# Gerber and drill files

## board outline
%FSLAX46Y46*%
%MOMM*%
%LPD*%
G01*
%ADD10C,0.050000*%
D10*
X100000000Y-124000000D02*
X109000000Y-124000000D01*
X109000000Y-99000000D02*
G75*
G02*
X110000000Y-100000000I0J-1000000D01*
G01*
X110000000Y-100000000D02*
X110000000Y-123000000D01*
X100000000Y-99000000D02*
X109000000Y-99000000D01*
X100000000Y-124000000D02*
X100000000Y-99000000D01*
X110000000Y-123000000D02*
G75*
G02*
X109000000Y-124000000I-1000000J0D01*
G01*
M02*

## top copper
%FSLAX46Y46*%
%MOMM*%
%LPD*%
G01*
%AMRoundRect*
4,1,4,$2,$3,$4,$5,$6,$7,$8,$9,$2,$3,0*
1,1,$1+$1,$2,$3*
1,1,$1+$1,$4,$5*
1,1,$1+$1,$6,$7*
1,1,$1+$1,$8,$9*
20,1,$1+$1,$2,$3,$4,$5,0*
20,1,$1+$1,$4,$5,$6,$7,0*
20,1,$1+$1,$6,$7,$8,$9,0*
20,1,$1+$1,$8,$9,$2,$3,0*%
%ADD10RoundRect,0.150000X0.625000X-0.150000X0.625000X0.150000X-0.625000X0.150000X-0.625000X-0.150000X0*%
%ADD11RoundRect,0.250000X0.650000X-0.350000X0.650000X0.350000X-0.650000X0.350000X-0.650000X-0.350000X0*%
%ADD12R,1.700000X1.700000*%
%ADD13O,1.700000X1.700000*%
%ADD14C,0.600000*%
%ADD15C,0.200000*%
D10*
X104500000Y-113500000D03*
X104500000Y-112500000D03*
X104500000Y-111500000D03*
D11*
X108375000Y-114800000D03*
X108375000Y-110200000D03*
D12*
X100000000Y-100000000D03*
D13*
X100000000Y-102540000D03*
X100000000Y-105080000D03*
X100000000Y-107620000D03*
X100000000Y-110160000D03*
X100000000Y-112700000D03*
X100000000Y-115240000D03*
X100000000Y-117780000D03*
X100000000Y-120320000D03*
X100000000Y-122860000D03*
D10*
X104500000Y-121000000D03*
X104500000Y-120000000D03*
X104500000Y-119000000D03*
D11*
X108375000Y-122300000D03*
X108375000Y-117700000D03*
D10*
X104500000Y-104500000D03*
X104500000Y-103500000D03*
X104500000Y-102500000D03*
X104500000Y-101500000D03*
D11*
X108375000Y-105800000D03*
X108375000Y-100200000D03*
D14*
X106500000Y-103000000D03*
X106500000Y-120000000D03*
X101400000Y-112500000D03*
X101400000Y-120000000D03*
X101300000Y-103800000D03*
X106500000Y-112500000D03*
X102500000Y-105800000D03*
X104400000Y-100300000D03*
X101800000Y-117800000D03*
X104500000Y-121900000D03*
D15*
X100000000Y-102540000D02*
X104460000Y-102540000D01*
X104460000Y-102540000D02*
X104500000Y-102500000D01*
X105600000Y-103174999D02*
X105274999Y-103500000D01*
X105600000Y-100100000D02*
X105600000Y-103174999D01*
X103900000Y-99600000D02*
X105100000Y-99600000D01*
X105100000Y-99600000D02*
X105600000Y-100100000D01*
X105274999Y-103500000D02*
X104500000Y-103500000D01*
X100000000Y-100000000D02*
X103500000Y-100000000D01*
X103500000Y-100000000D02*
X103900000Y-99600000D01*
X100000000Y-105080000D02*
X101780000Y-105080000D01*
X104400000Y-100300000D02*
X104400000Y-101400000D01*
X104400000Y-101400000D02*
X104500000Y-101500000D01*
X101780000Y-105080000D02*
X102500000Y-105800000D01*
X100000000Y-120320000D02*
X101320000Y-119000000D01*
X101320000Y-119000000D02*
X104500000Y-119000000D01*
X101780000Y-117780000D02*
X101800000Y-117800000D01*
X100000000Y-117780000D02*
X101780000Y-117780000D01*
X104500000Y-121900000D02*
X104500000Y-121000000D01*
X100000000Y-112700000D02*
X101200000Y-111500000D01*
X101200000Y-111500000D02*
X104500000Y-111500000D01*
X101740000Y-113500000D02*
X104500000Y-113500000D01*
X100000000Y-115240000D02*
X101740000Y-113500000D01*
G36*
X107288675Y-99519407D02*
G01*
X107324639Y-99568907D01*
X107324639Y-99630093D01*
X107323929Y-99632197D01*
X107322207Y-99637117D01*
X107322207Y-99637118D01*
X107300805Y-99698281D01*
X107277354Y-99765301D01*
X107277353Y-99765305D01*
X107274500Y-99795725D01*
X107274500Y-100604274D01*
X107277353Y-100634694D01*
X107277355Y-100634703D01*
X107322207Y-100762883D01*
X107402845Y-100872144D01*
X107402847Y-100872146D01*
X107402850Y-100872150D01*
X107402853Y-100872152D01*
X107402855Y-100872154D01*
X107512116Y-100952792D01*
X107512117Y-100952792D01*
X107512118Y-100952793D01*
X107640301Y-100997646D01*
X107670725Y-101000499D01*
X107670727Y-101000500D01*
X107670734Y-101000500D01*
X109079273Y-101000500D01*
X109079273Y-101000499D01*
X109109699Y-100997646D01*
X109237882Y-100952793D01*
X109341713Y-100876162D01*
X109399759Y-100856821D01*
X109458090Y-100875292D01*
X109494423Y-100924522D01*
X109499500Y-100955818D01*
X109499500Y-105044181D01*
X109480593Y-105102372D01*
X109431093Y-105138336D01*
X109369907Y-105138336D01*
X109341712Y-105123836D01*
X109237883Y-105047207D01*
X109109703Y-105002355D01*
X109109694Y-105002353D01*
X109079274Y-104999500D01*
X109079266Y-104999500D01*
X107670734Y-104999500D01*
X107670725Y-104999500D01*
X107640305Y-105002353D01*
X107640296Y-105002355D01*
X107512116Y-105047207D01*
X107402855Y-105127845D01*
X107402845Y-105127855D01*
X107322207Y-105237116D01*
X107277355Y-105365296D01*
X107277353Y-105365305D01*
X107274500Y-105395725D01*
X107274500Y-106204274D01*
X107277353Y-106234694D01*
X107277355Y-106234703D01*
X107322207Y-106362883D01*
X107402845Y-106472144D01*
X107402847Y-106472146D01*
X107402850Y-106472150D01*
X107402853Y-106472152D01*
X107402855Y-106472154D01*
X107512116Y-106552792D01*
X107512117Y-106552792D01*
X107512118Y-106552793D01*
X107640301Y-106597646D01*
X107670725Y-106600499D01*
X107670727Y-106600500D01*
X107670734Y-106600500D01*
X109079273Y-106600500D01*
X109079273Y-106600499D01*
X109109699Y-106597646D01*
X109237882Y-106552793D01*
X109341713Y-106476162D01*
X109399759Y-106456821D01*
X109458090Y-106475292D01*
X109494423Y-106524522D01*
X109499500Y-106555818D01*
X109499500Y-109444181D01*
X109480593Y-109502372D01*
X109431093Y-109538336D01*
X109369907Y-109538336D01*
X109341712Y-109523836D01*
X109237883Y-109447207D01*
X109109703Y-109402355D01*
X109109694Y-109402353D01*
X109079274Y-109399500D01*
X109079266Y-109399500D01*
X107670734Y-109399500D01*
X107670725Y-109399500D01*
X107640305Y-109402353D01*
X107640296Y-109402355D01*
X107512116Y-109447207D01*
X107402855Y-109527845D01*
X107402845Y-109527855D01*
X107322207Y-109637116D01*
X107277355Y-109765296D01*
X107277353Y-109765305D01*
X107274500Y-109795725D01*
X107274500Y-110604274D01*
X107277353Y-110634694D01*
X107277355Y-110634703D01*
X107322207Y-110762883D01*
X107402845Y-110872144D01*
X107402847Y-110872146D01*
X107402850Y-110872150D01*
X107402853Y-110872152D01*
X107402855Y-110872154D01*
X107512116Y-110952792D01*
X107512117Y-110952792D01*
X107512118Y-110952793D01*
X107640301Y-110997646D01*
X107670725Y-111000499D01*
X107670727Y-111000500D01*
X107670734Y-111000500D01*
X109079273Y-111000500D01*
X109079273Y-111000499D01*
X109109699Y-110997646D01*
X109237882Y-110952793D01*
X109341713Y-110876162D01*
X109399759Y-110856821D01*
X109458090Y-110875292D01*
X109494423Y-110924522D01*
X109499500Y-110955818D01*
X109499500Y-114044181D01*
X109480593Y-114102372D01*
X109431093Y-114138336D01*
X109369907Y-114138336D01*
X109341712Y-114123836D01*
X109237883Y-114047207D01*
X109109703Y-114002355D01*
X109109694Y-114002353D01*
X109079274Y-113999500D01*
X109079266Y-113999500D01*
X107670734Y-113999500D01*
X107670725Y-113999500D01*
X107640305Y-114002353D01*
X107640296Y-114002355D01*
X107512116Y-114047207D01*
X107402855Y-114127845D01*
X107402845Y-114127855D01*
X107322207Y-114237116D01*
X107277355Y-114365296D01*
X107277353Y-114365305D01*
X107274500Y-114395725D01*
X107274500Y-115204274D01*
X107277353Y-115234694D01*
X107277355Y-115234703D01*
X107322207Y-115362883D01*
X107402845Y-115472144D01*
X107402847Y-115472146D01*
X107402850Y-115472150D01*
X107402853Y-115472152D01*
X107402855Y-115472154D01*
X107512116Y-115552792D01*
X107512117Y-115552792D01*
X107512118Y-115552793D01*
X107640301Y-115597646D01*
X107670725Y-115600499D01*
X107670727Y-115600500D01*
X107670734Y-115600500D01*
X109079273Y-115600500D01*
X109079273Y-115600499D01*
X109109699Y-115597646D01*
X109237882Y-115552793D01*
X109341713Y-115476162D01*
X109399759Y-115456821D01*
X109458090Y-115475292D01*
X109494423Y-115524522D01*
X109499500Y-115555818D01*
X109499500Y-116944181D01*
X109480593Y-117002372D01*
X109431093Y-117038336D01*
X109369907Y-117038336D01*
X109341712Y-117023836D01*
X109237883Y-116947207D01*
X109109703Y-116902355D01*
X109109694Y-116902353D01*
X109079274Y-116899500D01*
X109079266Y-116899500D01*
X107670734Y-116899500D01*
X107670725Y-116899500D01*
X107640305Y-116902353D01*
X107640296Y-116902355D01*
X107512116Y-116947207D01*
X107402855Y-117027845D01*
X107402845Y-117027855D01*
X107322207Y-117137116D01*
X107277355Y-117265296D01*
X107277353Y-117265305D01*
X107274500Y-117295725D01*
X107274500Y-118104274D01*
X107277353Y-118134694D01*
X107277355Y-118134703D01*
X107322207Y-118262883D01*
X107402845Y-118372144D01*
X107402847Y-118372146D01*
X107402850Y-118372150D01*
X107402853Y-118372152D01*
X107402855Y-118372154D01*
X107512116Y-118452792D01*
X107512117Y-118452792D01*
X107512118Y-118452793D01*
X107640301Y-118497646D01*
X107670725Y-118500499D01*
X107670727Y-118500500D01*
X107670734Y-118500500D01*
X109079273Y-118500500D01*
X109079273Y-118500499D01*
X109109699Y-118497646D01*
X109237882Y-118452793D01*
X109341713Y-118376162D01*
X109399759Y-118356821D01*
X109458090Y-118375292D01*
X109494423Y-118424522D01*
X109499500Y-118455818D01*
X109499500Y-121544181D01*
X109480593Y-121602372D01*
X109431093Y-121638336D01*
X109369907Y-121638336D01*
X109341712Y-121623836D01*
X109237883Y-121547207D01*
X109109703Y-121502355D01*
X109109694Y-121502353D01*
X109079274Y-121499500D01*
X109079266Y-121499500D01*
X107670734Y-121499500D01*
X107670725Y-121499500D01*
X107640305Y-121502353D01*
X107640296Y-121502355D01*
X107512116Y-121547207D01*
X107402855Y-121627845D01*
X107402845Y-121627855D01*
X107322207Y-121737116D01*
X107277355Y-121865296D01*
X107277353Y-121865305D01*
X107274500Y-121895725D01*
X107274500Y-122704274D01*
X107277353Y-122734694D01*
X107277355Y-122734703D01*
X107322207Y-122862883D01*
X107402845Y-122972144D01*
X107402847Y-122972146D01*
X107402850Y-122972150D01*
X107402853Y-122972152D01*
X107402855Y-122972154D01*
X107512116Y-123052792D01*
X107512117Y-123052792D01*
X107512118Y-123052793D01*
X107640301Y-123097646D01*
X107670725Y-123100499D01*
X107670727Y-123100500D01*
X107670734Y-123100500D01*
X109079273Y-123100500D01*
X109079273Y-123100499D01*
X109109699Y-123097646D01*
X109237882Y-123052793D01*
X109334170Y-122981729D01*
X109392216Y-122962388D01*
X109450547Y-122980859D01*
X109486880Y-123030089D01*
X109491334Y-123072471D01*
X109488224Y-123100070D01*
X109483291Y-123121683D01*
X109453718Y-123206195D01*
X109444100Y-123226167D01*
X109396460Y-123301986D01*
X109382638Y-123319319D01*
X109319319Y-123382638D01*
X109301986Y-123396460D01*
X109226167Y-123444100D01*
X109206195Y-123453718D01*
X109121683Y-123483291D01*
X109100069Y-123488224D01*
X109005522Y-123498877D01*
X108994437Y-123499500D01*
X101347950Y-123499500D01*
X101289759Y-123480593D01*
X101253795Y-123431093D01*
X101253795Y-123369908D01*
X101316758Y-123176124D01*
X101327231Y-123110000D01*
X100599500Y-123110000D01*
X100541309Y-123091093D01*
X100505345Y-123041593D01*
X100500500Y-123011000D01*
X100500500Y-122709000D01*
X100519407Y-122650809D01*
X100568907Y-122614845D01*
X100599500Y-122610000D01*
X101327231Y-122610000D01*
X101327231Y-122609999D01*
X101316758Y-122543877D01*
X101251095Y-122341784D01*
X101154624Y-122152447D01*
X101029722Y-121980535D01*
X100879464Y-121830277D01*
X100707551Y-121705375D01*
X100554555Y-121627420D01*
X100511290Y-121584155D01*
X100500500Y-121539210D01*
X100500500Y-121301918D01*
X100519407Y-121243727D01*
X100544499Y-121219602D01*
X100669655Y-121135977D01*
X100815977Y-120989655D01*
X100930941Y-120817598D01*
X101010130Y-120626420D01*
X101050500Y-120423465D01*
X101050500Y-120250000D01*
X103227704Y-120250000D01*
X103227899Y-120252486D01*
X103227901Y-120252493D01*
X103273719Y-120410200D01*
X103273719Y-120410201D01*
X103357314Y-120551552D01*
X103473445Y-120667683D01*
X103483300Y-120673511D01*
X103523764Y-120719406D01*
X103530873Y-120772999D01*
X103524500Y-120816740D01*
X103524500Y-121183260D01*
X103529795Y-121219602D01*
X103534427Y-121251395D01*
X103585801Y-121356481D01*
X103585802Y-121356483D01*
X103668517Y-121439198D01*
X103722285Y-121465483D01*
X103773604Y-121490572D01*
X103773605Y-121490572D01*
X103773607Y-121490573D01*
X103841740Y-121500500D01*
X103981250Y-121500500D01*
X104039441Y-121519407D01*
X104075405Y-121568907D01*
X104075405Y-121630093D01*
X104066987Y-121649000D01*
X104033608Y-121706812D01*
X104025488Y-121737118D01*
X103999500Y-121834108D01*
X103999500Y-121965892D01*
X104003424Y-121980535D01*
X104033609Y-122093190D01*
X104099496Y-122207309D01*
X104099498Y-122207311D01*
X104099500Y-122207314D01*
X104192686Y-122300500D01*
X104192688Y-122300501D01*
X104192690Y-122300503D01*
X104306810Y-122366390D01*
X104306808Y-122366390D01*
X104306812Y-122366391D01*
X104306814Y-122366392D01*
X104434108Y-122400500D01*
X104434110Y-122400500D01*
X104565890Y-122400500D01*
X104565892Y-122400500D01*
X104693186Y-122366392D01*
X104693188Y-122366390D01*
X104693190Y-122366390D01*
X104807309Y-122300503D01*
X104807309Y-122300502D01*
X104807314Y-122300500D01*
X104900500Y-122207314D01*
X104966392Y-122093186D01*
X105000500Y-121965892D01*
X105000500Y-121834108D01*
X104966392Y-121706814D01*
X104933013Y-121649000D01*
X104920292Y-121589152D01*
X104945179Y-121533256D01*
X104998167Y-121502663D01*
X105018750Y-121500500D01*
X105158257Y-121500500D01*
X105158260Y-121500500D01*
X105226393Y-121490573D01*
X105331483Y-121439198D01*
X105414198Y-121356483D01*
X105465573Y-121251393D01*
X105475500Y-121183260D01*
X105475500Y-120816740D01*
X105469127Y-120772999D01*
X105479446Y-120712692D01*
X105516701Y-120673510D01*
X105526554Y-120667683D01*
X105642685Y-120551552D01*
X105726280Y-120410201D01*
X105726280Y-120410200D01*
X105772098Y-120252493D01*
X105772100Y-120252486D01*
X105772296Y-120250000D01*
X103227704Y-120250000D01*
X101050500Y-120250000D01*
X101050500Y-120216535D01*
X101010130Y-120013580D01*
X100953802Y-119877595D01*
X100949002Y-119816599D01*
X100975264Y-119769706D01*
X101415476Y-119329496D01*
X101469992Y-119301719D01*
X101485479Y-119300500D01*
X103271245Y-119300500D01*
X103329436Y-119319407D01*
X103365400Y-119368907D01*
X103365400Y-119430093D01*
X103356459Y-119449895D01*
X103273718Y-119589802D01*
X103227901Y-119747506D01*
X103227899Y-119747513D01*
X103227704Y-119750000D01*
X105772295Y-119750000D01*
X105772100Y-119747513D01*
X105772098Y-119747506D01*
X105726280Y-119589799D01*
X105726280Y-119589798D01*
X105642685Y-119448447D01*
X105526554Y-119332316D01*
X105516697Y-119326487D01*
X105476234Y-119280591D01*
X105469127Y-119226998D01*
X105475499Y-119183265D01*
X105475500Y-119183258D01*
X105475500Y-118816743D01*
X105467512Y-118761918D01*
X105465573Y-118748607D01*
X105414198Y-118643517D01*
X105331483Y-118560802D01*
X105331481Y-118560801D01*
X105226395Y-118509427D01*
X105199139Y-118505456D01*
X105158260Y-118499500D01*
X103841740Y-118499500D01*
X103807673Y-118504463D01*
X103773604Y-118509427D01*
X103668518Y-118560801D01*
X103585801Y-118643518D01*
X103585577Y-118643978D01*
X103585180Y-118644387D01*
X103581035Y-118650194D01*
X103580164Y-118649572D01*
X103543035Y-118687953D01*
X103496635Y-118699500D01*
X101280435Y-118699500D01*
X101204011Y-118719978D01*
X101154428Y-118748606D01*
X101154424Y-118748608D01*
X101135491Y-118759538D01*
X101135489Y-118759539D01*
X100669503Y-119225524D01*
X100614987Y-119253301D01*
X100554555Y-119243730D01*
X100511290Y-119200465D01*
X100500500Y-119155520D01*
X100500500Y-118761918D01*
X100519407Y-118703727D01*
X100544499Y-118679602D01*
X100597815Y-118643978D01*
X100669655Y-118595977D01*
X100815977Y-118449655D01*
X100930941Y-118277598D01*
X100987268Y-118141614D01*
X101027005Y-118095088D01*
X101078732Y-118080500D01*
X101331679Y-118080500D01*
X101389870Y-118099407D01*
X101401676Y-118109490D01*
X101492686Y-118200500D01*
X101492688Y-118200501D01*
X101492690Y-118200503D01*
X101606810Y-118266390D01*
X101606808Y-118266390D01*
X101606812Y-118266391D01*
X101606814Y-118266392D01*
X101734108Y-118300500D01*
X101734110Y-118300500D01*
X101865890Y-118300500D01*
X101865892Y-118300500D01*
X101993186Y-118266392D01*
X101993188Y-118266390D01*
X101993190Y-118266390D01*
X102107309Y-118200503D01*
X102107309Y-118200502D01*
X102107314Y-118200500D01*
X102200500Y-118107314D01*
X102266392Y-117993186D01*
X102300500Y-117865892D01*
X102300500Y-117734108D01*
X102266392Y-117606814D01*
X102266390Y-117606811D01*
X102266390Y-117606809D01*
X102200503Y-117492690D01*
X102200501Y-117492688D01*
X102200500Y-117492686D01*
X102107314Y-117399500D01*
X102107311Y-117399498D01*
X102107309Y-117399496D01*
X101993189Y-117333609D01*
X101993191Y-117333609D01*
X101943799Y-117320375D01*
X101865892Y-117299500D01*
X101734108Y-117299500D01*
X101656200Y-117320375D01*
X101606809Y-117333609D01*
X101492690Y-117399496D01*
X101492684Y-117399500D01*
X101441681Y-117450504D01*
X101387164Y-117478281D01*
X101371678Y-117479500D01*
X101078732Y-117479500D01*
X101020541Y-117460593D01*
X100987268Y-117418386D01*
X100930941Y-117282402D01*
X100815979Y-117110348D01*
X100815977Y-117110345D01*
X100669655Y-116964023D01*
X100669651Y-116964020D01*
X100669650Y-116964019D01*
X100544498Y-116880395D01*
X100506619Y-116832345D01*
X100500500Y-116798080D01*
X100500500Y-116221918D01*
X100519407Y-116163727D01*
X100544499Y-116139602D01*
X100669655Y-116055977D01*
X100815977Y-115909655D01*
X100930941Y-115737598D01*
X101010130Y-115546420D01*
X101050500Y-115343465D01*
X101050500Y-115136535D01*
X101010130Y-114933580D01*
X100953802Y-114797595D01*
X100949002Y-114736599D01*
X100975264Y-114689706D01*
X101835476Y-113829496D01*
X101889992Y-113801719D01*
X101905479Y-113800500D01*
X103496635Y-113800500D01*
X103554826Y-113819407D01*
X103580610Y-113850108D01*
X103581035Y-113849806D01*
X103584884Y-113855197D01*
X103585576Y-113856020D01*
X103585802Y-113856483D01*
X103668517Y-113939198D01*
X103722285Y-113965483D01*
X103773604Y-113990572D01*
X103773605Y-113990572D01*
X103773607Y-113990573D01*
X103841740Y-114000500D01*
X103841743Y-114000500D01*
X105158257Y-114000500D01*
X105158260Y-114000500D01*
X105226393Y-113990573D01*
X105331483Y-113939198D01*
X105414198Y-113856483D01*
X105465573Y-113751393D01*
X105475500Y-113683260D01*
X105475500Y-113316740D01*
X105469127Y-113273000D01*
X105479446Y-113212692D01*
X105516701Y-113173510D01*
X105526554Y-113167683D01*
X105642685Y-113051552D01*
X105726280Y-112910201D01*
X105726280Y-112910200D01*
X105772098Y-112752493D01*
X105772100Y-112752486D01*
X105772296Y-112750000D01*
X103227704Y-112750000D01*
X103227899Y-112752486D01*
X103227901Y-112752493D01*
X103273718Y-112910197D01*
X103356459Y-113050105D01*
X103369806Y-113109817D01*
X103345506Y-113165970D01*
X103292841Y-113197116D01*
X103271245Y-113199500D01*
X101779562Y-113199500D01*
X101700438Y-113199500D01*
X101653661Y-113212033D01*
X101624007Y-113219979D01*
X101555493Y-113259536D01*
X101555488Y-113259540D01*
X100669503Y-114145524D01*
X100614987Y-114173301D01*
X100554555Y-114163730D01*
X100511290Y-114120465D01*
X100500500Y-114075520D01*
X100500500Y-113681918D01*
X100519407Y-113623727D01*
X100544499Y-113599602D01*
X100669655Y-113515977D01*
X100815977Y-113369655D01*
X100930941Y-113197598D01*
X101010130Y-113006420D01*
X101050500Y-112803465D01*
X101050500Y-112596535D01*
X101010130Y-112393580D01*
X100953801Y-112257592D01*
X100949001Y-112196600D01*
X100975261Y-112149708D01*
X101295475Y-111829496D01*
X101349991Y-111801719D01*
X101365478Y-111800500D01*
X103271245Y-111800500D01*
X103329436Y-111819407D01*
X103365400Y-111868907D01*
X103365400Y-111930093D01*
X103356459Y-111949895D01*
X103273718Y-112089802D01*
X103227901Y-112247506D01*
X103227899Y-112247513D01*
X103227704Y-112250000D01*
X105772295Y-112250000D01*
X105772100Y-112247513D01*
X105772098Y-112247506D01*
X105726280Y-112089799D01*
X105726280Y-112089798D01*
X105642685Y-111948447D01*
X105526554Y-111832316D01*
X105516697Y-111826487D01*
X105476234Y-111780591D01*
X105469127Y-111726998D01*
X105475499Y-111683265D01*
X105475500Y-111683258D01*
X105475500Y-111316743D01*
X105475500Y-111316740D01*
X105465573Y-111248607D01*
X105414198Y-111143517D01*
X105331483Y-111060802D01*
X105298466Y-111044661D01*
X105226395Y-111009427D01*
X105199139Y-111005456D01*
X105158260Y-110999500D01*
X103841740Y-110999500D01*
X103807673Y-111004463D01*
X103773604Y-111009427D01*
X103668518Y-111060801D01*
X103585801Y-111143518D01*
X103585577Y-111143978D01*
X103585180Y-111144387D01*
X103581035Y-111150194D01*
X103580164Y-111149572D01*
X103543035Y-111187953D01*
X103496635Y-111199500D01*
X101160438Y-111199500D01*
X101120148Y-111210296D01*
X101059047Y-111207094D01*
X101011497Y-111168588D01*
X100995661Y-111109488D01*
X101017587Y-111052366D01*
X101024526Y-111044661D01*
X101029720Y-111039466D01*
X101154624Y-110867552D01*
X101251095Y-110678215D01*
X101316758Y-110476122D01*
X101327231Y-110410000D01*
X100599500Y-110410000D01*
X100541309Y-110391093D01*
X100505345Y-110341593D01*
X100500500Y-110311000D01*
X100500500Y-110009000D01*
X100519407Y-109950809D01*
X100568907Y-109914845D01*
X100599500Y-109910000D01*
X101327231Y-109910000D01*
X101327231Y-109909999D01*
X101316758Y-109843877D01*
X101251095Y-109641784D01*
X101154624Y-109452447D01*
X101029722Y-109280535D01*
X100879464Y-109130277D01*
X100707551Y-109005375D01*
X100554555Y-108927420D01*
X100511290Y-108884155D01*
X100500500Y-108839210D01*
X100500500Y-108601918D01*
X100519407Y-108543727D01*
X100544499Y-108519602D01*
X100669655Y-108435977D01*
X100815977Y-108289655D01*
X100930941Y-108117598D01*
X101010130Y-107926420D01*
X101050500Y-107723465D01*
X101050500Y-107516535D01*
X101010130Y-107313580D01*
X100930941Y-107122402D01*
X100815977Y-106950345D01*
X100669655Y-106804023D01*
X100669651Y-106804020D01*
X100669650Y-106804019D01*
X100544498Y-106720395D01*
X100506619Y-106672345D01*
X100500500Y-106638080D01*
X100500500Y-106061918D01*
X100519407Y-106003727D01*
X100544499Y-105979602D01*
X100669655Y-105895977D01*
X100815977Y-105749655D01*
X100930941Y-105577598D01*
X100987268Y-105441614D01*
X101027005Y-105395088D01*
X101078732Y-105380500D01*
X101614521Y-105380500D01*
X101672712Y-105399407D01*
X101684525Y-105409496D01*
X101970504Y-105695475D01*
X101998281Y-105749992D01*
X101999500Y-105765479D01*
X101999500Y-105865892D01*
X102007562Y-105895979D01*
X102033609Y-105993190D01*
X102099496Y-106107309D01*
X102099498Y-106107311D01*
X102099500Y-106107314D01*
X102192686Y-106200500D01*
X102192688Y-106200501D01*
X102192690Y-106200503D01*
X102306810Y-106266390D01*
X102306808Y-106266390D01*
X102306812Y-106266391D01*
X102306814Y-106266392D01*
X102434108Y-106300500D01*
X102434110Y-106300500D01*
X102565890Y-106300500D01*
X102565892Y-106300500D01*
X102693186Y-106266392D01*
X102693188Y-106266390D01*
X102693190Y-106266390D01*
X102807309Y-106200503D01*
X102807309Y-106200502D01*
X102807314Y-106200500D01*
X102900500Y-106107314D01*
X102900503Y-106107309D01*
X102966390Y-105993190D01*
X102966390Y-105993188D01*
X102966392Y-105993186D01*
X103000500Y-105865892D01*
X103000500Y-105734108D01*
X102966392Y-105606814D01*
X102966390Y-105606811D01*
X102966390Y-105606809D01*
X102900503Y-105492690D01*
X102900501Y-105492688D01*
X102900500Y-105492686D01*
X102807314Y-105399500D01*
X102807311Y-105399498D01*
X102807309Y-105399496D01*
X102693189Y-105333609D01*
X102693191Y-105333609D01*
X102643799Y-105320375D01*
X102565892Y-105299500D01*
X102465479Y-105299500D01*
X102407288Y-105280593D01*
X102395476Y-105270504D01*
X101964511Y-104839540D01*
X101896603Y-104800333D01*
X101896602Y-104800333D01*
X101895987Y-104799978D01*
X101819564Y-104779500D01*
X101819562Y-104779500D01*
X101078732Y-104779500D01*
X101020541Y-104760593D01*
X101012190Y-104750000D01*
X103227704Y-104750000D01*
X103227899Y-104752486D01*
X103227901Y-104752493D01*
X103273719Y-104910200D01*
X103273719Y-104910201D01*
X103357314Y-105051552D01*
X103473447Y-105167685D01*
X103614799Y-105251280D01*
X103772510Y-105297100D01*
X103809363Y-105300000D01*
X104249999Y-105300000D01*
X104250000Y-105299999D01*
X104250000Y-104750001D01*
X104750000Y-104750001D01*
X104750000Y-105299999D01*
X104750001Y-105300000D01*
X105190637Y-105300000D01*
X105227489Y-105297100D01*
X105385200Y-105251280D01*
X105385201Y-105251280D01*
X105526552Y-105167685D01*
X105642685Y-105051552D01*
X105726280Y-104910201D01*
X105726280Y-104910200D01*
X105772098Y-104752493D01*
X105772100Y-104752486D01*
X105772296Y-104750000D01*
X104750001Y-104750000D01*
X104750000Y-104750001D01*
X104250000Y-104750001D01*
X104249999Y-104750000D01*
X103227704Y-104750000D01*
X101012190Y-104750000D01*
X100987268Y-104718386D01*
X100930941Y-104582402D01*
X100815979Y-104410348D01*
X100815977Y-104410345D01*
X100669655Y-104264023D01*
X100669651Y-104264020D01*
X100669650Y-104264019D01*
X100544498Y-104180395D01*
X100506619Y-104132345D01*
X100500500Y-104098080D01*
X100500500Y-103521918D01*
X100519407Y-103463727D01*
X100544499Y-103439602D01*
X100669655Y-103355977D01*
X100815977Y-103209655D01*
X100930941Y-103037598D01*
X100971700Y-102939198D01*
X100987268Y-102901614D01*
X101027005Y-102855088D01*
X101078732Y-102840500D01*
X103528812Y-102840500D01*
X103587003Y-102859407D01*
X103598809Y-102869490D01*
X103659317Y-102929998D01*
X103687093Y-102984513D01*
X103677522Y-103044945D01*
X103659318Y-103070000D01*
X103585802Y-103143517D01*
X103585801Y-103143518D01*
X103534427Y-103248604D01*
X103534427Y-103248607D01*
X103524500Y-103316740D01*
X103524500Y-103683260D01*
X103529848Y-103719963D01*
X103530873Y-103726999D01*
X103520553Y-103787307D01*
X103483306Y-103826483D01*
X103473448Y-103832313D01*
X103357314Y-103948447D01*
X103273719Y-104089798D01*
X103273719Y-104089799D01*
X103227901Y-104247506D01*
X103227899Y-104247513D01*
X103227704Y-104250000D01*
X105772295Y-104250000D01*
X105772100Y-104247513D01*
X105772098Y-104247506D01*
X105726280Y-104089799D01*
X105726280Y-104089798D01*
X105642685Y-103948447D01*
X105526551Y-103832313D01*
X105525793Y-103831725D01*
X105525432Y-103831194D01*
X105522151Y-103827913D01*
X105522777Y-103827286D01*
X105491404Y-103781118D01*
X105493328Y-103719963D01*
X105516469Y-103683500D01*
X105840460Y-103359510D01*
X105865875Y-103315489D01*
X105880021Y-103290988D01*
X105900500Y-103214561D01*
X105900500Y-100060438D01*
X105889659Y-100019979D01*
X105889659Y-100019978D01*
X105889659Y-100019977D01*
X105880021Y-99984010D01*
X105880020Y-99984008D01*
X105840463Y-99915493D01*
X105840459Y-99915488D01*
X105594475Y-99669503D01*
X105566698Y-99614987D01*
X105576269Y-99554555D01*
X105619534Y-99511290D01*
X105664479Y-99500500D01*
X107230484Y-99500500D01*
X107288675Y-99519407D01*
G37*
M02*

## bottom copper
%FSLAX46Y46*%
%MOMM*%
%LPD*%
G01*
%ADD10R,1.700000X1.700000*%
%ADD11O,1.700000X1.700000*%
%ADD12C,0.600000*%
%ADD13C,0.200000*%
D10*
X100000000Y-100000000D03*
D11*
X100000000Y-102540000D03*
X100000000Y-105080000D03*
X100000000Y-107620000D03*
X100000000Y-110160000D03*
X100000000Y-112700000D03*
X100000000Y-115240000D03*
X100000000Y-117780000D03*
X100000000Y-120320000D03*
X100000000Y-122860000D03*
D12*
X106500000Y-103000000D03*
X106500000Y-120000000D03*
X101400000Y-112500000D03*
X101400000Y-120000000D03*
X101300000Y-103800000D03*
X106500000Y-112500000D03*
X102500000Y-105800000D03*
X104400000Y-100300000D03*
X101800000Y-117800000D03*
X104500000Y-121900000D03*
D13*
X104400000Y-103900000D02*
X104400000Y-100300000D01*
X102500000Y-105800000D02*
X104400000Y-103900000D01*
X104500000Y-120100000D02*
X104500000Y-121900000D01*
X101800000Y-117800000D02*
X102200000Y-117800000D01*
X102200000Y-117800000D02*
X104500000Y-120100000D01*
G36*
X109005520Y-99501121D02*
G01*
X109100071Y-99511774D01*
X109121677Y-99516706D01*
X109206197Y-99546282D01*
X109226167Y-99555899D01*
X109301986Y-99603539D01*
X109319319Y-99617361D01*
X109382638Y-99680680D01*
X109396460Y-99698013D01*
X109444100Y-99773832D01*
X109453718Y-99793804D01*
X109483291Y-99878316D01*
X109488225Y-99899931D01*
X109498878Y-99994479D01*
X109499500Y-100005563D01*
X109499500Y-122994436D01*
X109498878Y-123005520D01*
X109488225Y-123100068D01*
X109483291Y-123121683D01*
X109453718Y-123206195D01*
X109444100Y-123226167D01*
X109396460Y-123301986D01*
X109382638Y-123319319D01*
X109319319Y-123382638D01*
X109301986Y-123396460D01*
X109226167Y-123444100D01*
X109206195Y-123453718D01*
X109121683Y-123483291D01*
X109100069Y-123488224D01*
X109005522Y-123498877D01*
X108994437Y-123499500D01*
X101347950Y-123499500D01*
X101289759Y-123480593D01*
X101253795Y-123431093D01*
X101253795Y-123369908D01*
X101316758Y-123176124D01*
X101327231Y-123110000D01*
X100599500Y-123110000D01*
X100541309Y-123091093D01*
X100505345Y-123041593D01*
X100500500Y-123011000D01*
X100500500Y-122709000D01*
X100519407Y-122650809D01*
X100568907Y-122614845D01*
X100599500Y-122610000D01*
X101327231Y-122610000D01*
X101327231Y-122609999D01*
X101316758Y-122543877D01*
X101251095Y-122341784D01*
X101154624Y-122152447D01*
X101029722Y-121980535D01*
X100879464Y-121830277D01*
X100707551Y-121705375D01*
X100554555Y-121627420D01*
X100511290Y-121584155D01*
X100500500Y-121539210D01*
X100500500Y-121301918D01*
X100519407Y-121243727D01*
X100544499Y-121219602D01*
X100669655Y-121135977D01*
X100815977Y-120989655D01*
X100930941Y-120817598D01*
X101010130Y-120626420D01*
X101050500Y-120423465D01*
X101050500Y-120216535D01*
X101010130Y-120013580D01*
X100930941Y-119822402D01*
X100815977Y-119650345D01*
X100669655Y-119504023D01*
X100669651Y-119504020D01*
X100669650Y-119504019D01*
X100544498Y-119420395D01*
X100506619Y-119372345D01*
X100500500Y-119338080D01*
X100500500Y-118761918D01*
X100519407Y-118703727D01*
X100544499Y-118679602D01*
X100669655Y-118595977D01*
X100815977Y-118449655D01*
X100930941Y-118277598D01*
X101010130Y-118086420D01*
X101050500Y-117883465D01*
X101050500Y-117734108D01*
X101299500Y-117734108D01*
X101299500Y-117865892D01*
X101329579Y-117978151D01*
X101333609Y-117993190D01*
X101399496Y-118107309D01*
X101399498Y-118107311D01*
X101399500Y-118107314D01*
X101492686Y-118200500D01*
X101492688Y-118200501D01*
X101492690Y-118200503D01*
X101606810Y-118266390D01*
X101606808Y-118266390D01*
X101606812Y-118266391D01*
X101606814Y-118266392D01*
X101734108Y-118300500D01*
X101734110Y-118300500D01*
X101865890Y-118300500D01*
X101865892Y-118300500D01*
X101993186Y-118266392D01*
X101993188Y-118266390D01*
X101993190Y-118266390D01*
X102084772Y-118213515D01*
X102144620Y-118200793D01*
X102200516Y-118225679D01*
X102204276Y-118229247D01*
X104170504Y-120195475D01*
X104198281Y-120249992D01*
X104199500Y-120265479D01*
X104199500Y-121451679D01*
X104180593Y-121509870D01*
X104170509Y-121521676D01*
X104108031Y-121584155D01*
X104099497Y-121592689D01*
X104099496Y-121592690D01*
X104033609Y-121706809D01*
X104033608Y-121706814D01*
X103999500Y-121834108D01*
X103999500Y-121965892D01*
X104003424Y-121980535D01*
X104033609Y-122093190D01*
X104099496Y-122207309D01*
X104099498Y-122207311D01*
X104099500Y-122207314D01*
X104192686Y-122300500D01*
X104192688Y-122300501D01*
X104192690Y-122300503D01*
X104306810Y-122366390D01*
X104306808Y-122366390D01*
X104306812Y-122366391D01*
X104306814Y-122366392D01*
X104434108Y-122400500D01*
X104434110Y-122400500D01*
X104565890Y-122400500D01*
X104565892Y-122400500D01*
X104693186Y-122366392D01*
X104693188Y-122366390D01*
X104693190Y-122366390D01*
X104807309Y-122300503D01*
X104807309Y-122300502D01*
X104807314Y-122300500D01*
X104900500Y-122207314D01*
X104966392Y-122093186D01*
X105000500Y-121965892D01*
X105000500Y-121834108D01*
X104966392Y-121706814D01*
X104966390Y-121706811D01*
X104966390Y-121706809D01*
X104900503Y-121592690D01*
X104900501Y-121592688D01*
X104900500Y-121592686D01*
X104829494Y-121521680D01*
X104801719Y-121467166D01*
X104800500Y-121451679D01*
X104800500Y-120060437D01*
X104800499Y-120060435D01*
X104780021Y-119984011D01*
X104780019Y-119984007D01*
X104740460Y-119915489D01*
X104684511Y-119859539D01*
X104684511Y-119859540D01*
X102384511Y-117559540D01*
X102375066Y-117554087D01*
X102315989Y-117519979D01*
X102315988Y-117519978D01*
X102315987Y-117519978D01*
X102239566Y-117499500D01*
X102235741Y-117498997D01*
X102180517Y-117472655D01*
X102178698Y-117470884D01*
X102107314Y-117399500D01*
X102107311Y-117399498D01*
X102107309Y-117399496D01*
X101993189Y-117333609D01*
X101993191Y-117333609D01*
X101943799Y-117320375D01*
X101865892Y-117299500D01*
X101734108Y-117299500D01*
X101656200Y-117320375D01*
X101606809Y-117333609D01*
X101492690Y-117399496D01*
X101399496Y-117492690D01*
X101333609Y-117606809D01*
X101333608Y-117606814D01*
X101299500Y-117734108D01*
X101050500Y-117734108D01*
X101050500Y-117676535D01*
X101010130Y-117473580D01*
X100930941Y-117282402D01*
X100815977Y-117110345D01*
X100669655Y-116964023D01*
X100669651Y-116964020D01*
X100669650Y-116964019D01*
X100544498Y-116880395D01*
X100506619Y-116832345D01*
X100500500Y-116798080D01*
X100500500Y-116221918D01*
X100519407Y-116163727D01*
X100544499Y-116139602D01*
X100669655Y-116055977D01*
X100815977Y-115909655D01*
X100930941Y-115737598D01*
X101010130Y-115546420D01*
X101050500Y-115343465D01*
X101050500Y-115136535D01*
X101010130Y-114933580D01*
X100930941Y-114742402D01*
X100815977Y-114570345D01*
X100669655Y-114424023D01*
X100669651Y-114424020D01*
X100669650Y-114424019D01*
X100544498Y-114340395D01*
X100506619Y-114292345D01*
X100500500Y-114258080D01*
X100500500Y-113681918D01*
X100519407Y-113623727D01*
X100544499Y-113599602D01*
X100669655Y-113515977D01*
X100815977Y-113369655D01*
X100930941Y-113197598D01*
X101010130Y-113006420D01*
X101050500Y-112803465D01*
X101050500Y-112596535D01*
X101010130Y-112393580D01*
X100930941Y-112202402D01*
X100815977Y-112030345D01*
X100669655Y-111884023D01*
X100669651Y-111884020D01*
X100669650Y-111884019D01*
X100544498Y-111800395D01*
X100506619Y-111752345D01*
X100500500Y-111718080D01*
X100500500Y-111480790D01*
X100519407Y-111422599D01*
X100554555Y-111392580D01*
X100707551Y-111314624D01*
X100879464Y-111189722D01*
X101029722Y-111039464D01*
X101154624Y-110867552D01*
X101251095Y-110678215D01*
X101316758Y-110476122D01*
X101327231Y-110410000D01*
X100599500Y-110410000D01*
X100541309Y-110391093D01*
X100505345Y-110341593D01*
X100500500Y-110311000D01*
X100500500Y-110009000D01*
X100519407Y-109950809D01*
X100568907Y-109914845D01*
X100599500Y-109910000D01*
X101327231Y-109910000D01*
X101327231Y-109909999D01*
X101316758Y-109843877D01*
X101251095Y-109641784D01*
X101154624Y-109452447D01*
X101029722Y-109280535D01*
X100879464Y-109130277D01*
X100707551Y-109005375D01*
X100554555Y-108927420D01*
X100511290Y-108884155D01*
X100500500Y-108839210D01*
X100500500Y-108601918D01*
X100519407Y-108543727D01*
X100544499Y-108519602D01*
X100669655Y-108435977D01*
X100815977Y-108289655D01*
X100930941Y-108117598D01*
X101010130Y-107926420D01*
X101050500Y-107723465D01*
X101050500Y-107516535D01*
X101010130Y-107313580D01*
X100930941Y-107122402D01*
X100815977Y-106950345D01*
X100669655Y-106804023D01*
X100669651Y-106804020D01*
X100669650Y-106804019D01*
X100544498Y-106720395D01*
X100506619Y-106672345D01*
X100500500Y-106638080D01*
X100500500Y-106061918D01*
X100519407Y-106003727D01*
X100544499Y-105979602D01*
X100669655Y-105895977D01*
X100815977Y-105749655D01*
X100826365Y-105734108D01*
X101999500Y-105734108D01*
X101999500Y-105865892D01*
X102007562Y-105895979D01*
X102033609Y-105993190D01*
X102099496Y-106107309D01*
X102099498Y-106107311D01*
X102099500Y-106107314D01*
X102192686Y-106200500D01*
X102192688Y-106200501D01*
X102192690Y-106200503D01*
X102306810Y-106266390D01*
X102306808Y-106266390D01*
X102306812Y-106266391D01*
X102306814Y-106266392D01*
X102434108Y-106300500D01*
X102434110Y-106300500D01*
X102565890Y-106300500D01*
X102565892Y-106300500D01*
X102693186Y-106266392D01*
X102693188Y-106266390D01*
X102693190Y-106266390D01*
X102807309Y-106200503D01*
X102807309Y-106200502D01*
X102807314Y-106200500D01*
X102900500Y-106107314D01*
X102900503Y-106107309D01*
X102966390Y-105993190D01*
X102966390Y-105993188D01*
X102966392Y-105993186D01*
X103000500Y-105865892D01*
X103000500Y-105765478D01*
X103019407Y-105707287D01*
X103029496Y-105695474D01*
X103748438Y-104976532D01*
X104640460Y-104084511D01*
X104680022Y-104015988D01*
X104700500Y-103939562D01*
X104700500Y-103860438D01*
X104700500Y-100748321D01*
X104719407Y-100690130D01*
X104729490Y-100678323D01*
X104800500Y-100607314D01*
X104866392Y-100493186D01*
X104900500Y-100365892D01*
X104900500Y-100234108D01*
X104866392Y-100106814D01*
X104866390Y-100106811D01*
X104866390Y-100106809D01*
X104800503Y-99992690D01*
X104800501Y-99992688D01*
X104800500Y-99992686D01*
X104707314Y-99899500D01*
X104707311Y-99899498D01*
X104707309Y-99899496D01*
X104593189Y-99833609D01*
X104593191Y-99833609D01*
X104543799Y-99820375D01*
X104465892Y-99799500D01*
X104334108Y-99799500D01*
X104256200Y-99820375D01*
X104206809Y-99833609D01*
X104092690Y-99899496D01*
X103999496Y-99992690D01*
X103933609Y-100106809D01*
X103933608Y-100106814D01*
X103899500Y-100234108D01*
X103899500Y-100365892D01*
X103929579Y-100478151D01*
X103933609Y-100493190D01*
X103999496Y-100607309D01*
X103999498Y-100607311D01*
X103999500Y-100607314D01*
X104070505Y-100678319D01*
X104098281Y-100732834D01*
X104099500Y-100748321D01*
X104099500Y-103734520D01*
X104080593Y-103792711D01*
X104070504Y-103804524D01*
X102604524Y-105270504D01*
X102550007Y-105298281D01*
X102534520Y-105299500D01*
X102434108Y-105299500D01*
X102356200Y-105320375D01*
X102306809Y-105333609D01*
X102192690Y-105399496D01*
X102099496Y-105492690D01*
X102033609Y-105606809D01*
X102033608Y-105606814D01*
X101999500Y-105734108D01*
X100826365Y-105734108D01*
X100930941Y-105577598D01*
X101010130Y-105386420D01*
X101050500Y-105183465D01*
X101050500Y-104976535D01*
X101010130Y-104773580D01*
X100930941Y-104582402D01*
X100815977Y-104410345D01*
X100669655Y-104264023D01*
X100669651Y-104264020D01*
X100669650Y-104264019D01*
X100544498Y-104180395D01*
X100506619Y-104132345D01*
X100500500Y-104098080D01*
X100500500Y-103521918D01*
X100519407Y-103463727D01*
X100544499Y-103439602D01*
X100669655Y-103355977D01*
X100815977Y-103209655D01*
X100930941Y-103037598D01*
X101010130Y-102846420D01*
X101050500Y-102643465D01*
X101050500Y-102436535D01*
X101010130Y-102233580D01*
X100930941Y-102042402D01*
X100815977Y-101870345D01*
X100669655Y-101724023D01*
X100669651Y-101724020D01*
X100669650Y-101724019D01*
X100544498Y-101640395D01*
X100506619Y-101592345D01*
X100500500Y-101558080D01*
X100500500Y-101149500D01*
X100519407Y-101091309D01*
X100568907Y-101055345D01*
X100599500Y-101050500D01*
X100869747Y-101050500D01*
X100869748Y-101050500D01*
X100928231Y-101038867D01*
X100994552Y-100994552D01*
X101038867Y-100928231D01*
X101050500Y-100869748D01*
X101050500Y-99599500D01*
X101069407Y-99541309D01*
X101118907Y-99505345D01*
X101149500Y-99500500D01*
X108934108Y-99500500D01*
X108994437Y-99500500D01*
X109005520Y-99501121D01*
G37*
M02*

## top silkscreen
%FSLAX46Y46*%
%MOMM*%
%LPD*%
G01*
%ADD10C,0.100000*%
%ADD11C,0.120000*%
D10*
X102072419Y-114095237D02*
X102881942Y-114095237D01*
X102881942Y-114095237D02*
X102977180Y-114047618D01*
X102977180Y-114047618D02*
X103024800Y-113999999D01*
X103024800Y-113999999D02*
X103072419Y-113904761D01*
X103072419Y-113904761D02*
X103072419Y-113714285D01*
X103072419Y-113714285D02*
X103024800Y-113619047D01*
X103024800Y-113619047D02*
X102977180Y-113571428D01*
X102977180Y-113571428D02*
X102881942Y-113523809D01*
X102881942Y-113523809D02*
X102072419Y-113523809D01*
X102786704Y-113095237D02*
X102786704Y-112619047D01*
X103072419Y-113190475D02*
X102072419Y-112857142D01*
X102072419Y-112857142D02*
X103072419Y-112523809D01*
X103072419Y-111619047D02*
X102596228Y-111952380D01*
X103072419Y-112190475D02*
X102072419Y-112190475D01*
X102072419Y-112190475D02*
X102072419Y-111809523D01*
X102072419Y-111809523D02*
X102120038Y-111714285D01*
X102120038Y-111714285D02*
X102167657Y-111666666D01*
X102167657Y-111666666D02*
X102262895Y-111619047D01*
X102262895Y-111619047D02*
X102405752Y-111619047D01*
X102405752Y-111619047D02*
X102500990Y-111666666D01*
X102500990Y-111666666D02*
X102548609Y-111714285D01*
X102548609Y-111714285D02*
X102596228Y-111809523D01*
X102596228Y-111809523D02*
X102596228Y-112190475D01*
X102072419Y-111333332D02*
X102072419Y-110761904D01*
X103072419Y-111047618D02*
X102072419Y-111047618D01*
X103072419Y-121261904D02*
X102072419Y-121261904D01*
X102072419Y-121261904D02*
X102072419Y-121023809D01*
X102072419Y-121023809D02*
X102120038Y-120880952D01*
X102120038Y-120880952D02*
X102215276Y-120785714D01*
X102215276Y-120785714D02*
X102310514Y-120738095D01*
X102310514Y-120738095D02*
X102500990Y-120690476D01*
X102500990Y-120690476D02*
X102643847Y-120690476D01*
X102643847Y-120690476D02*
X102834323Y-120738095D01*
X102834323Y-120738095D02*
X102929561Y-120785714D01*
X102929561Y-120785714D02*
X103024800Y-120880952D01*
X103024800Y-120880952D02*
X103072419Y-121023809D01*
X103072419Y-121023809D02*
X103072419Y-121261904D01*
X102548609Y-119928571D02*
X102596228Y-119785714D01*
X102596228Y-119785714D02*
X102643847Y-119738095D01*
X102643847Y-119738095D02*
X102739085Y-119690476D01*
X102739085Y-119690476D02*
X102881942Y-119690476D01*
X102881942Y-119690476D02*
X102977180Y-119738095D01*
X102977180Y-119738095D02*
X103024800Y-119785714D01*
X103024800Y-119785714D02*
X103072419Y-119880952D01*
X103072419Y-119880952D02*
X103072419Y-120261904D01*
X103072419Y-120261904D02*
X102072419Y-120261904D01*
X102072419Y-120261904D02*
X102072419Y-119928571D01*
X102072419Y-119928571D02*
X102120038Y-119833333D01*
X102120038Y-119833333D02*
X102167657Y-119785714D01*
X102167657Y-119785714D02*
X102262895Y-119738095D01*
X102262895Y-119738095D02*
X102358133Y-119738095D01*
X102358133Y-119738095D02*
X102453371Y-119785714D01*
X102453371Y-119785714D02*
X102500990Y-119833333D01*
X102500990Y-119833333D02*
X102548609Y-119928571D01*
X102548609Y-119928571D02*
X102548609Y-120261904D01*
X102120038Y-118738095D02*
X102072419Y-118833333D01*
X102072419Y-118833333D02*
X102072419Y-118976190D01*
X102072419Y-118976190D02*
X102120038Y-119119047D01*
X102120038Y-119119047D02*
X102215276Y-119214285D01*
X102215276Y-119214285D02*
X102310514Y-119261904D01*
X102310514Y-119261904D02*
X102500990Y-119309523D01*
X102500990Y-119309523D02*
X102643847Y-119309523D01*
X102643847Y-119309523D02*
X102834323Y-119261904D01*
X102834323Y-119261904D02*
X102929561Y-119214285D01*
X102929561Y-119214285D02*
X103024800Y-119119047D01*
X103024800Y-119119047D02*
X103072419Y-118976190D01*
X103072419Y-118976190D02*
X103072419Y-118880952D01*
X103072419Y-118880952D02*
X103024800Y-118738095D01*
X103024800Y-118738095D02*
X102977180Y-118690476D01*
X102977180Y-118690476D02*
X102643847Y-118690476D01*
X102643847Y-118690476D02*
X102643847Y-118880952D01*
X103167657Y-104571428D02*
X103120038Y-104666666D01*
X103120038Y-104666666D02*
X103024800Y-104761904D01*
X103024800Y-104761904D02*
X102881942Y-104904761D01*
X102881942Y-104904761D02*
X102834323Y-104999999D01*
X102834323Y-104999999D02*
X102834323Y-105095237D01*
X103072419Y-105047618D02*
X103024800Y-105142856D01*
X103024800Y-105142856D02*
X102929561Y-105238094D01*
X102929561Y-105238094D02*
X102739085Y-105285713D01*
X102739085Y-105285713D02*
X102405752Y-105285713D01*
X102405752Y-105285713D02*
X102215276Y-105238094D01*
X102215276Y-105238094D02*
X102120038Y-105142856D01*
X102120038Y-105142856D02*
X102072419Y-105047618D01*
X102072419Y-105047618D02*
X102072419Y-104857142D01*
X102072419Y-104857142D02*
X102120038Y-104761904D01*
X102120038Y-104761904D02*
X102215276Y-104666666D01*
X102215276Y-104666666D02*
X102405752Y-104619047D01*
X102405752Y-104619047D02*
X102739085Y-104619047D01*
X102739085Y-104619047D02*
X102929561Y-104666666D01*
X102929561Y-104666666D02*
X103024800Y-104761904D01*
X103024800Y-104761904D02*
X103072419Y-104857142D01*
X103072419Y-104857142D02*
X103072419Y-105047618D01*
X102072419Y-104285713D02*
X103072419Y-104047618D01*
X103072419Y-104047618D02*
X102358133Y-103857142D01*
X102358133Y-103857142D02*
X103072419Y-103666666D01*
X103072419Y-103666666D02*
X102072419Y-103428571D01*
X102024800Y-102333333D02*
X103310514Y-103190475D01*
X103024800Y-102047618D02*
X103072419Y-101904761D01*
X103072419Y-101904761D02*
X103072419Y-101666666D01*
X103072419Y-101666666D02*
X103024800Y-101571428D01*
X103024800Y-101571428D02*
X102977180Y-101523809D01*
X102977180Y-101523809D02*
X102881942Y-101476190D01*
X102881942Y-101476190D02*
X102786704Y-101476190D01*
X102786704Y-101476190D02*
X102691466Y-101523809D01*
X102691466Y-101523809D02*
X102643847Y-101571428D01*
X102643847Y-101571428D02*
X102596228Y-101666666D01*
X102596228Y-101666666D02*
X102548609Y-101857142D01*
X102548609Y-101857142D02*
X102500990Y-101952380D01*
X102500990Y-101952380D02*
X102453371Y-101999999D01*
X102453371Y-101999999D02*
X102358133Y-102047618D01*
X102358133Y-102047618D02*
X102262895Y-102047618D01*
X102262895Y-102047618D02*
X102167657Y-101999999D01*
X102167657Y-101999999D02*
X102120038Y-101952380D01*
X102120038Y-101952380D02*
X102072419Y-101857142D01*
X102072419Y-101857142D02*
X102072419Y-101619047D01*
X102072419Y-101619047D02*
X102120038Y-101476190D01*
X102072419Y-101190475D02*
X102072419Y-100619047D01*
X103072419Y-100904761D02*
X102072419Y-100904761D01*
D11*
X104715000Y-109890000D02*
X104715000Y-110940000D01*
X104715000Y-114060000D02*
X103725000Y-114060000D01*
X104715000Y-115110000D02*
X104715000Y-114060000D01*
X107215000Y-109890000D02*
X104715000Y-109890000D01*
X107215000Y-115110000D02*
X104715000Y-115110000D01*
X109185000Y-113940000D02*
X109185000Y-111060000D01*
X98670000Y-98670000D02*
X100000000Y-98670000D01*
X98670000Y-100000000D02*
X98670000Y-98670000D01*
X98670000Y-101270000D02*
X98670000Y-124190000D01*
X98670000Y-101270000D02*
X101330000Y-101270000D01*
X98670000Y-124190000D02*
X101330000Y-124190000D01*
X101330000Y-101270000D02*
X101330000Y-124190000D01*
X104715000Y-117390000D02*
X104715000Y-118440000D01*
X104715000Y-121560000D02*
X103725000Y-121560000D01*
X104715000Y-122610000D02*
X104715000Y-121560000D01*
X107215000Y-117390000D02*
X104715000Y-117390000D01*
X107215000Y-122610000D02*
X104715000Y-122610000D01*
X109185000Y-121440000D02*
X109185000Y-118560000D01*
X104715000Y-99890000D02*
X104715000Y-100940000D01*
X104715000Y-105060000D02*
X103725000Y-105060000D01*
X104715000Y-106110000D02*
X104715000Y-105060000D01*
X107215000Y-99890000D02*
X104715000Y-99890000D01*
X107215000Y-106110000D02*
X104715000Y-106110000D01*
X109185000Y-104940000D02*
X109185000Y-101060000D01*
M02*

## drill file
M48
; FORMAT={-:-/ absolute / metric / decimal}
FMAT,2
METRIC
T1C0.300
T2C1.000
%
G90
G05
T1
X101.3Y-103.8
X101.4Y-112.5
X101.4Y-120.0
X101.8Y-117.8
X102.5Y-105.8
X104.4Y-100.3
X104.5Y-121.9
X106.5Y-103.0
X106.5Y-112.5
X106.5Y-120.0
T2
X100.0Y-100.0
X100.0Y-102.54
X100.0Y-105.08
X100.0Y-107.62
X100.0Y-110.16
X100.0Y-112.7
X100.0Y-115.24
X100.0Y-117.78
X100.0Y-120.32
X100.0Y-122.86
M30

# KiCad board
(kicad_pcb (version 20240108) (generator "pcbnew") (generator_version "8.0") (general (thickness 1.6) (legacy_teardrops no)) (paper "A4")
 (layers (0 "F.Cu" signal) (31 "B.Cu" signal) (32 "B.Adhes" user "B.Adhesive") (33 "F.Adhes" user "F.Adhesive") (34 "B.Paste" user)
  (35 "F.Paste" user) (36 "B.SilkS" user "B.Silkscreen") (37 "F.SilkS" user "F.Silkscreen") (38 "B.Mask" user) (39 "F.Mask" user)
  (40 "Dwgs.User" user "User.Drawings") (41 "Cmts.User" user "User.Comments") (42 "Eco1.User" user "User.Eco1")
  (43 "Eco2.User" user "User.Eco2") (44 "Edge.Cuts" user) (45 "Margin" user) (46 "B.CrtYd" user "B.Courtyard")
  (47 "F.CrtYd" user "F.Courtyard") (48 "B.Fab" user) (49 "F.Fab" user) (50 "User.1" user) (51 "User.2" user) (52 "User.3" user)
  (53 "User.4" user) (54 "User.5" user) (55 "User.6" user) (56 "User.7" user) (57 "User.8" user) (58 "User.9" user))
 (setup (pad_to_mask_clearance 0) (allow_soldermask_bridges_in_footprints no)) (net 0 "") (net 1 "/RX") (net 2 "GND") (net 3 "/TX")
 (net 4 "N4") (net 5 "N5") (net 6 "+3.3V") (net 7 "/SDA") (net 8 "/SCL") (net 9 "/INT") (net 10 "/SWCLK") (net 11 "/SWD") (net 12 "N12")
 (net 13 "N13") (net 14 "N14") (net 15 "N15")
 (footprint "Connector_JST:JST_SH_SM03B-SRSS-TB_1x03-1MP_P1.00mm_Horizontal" (layer "F.Cu") (at 106.5 112.5 90)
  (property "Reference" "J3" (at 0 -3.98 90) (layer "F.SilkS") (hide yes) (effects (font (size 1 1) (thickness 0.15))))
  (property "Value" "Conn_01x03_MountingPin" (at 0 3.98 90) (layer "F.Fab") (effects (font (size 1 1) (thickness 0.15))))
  (fp_line (start 2.61 -1.785) (end 1.56 -1.785) (stroke (width 0.12) (type solid)) (layer "F.SilkS"))
  (fp_line (start -1.56 -1.785) (end -1.56 -2.775) (stroke (width 0.12) (type solid)) (layer "F.SilkS"))
  (fp_line (start -2.61 -1.785) (end -1.56 -1.785) (stroke (width 0.12) (type solid)) (layer "F.SilkS"))
  (fp_line (start 2.61 0.715) (end 2.61 -1.785) (stroke (width 0.12) (type solid)) (layer "F.SilkS"))
  (fp_line (start -2.61 0.715) (end -2.61 -1.785) (stroke (width 0.12) (type solid)) (layer "F.SilkS"))
  (fp_line (start -1.44 2.685) (end 1.44 2.685) (stroke (width 0.12) (type solid)) (layer "F.SilkS"))
  (pad "1" smd roundrect (at -1 -2 90) (size 0.6 1.55) (layers "F.Cu" "F.Paste" "F.Mask") (roundrect_rratio 0.25) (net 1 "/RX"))
  (pad "2" smd roundrect (at 0 -2 90) (size 0.6 1.55) (layers "F.Cu" "F.Paste" "F.Mask") (roundrect_rratio 0.25) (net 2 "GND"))
  (pad "3" smd roundrect (at 1 -2 90) (size 0.6 1.55) (layers "F.Cu" "F.Paste" "F.Mask") (roundrect_rratio 0.25) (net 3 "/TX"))
  (pad "MP" smd roundrect (at -2.3 1.875 90) (size 1.2 1.8) (layers "F.Cu" "F.Paste" "F.Mask") (roundrect_rratio 0.208333) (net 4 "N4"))
  (pad "MP" smd roundrect (at 2.3 1.875 90) (size 1.2 1.8) (layers "F.Cu" "F.Paste" "F.Mask") (roundrect_rratio 0.208333) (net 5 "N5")))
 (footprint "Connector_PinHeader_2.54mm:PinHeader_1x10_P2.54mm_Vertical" (layer "F.Cu") (at 100 100)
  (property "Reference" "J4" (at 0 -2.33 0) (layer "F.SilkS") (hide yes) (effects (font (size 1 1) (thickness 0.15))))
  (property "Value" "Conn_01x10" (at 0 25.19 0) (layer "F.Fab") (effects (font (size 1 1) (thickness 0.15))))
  (fp_line (start -1.33 -1.33) (end 0 -1.33) (stroke (width 0.12) (type solid)) (layer "F.SilkS"))
  (fp_line (start -1.33 0) (end -1.33 -1.33) (stroke (width 0.12) (type solid)) (layer "F.SilkS"))
  (fp_line (start -1.33 1.27) (end -1.33 24.19) (stroke (width 0.12) (type solid)) (layer "F.SilkS"))
  (fp_line (start -1.33 1.27) (end 1.33 1.27) (stroke (width 0.12) (type solid)) (layer "F.SilkS"))
  (fp_line (start -1.33 24.19) (end 1.33 24.19) (stroke (width 0.12) (type solid)) (layer "F.SilkS"))
  (fp_line (start 1.33 1.27) (end 1.33 24.19) (stroke (width 0.12) (type solid)) (layer "F.SilkS"))
  (pad "1" thru_hole rect (at 0 0) (size 1.7 1.7) (drill 1) (layers "*.Cu" "*.Mask") (remove_unused_layers no) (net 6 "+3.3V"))
  (pad "2" thru_hole oval (at 0 2.54) (size 1.7 1.7) (drill 1) (layers "*.Cu" "*.Mask") (remove_unused_layers no) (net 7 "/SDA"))
  (pad "3" thru_hole oval (at 0 5.08) (size 1.7 1.7) (drill 1) (layers "*.Cu" "*.Mask") (remove_unused_layers no) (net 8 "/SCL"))
  (pad "4" thru_hole oval (at 0 7.62) (size 1.7 1.7) (drill 1) (layers "*.Cu" "*.Mask") (remove_unused_layers no) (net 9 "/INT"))
  (pad "5" thru_hole oval (at 0 10.16) (size 1.7 1.7) (drill 1) (layers "*.Cu" "*.Mask") (remove_unused_layers no) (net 2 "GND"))
  (pad "6" thru_hole oval (at 0 12.7) (size 1.7 1.7) (drill 1) (layers "*.Cu" "*.Mask") (remove_unused_layers no) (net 3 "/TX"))
  (pad "7" thru_hole oval (at 0 15.24) (size 1.7 1.7) (drill 1) (layers "*.Cu" "*.Mask") (remove_unused_layers no) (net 1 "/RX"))
  (pad "8" thru_hole oval (at 0 17.78) (size 1.7 1.7) (drill 1) (layers "*.Cu" "*.Mask") (remove_unused_layers no) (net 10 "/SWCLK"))
  (pad "9" thru_hole oval (at 0 20.32) (size 1.7 1.7) (drill 1) (layers "*.Cu" "*.Mask") (remove_unused_layers no) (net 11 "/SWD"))
  (pad "10" thru_hole oval (at 0 22.86) (size 1.7 1.7) (drill 1) (layers "*.Cu" "*.Mask") (remove_unused_layers no) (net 2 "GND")))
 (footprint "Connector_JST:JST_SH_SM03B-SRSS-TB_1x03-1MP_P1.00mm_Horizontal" (layer "F.Cu") (at 106.5 120 90)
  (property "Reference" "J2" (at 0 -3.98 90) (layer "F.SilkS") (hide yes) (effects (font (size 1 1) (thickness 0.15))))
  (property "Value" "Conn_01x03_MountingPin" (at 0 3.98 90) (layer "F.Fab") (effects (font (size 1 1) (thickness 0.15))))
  (fp_line (start 2.61 -1.785) (end 1.56 -1.785) (stroke (width 0.12) (type solid)) (layer "F.SilkS"))
  (fp_line (start -1.56 -1.785) (end -1.56 -2.775) (stroke (width 0.12) (type solid)) (layer "F.SilkS"))
  (fp_line (start -2.61 -1.785) (end -1.56 -1.785) (stroke (width 0.12) (type solid)) (layer "F.SilkS"))
  (fp_line (start 2.61 0.715) (end 2.61 -1.785) (stroke (width 0.12) (type solid)) (layer "F.SilkS"))
  (fp_line (start -2.61 0.715) (end -2.61 -1.785) (stroke (width 0.12) (type solid)) (layer "F.SilkS"))
  (fp_line (start -1.44 2.685) (end 1.44 2.685) (stroke (width 0.12) (type solid)) (layer "F.SilkS"))
  (pad "1" smd roundrect (at -1 -2 90) (size 0.6 1.55) (layers "F.Cu" "F.Paste" "F.Mask") (roundrect_rratio 0.25) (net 10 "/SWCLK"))
  (pad "2" smd roundrect (at 0 -2 90) (size 0.6 1.55) (layers "F.Cu" "F.Paste" "F.Mask") (roundrect_rratio 0.25) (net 2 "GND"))
  (pad "3" smd roundrect (at 1 -2 90) (size 0.6 1.55) (layers "F.Cu" "F.Paste" "F.Mask") (roundrect_rratio 0.25) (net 11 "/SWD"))
  (pad "MP" smd roundrect (at -2.3 1.875 90) (size 1.2 1.8) (layers "F.Cu" "F.Paste" "F.Mask") (roundrect_rratio 0.208333) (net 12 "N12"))
  (pad "MP" smd roundrect (at 2.3 1.875 90) (size 1.2 1.8) (layers "F.Cu" "F.Paste" "F.Mask") (roundrect_rratio 0.208333) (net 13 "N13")))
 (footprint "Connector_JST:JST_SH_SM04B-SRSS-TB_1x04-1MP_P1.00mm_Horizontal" (layer "F.Cu") (at 106.5 103 90)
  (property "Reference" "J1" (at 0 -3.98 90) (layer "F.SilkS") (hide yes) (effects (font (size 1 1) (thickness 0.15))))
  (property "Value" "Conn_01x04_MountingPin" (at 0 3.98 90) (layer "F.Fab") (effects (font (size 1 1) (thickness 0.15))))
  (fp_line (start 3.11 -1.785) (end 2.06 -1.785) (stroke (width 0.12) (type solid)) (layer "F.SilkS"))
  (fp_line (start -2.06 -1.785) (end -2.06 -2.775) (stroke (width 0.12) (type solid)) (layer "F.SilkS"))
  (fp_line (start -3.11 -1.785) (end -2.06 -1.785) (stroke (width 0.12) (type solid)) (layer "F.SilkS"))
  (fp_line (start 3.11 0.715) (end 3.11 -1.785) (stroke (width 0.12) (type solid)) (layer "F.SilkS"))
  (fp_line (start -3.11 0.715) (end -3.11 -1.785) (stroke (width 0.12) (type solid)) (layer "F.SilkS"))
  (fp_line (start -1.94 2.685) (end 1.94 2.685) (stroke (width 0.12) (type solid)) (layer "F.SilkS"))
  (pad "1" smd roundrect (at -1.5 -2 90) (size 0.6 1.55) (layers "F.Cu" "F.Paste" "F.Mask") (roundrect_rratio 0.25) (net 2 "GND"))
  (pad "2" smd roundrect (at -0.5 -2 90) (size 0.6 1.55) (layers "F.Cu" "F.Paste" "F.Mask") (roundrect_rratio 0.25) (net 6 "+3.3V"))
  (pad "3" smd roundrect (at 0.5 -2 90) (size 0.6 1.55) (layers "F.Cu" "F.Paste" "F.Mask") (roundrect_rratio 0.25) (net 7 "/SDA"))
  (pad "4" smd roundrect (at 1.5 -2 90) (size 0.6 1.55) (layers "F.Cu" "F.Paste" "F.Mask") (roundrect_rratio 0.25) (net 8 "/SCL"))
  (pad "MP" smd roundrect (at -2.8 1.875 90) (size 1.2 1.8) (layers "F.Cu" "F.Paste" "F.Mask") (roundrect_rratio 0.208333) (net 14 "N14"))
  (pad "MP" smd roundrect (at 2.8 1.875 90) (size 1.2 1.8) (layers "F.Cu" "F.Paste" "F.Mask") (roundrect_rratio 0.208333) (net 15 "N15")))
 (gr_line (start 100 124) (end 109 124) (stroke (width 0.05) (type default)) (layer "Edge.Cuts"))
 (gr_arc (start 109 99) (mid 109.707107 99.292893) (end 110 100) (stroke (width 0.05) (type default)) (layer "Edge.Cuts"))
 (gr_line (start 110 100) (end 110 123) (stroke (width 0.05) (type default)) (layer "Edge.Cuts"))
 (gr_line (start 100 99) (end 109 99) (stroke (width 0.05) (type default)) (layer "Edge.Cuts"))
 (gr_line (start 100 124) (end 100 99) (stroke (width 0.05) (type default)) (layer "Edge.Cuts"))
 (gr_arc (start 110 123) (mid 109.707107 123.707107) (end 109 124) (stroke (width 0.05) (type default)) (layer "Edge.Cuts"))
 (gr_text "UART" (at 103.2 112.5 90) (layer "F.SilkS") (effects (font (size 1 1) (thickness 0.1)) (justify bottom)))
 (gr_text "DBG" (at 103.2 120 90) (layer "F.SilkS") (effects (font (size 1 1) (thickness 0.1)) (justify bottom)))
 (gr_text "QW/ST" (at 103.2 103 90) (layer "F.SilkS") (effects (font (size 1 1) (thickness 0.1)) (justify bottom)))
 (via (at 106.5 103) (size 0.6) (drill 0.3) (layers "F.Cu" "B.Cu") (free yes) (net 2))
 (via (at 106.5 120) (size 0.6) (drill 0.3) (layers "F.Cu" "B.Cu") (free yes) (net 2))
 (via (at 101.4 112.5) (size 0.6) (drill 0.3) (layers "F.Cu" "B.Cu") (free yes) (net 2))
 (via (at 101.4 120) (size 0.6) (drill 0.3) (layers "F.Cu" "B.Cu") (free yes) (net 2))
 (via (at 101.3 103.8) (size 0.6) (drill 0.3) (layers "F.Cu" "B.Cu") (free yes) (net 2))
 (via (at 106.5 112.5) (size 0.6) (drill 0.3) (layers "F.Cu" "B.Cu") (free yes) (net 2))
 (segment (start 100 102.54) (end 104.46 102.54) (width 0.2) (layer "F.Cu") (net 7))
 (segment (start 104.46 102.54) (end 104.5 102.5) (width 0.2) (layer "F.Cu") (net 7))
 (segment (start 105.6 103.174999) (end 105.274999 103.5) (width 0.2) (layer "F.Cu") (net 6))
 (segment (start 105.6 100.1) (end 105.6 103.174999) (width 0.2) (layer "F.Cu") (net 6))
 (segment (start 103.9 99.6) (end 105.1 99.6) (width 0.2) (layer "F.Cu") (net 6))
 (segment (start 105.1 99.6) (end 105.6 100.1) (width 0.2) (layer "F.Cu") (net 6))
 (segment (start 105.274999 103.5) (end 104.5 103.5) (width 0.2) (layer "F.Cu") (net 6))
 (segment (start 100 100) (end 103.5 100) (width 0.2) (layer "F.Cu") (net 6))
 (segment (start 103.5 100) (end 103.9 99.6) (width 0.2) (layer "F.Cu") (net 6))
 (segment (start 100 105.08) (end 101.78 105.08) (width 0.2) (layer "F.Cu") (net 8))
 (segment (start 104.4 100.3) (end 104.4 101.4) (width 0.2) (layer "F.Cu") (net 8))
 (segment (start 104.4 101.4) (end 104.5 101.5) (width 0.2) (layer "F.Cu") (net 8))
 (segment (start 101.78 105.08) (end 102.5 105.8) (width 0.2) (layer "F.Cu") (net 8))
 (via (at 102.5 105.8) (size 0.6) (drill 0.3) (layers "F.Cu" "B.Cu") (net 8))
 (via (at 104.4 100.3) (size 0.6) (drill 0.3) (layers "F.Cu" "B.Cu") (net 8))
 (segment (start 104.4 103.9) (end 104.4 100.3) (width 0.2) (layer "B.Cu") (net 8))
 (segment (start 102.5 105.8) (end 104.4 103.9) (width 0.2) (layer "B.Cu") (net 8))
 (segment (start 100 120.32) (end 101.32 119) (width 0.2) (layer "F.Cu") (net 11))
 (segment (start 101.32 119) (end 104.5 119) (width 0.2) (layer "F.Cu") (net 11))
 (segment (start 101.78 117.78) (end 101.8 117.8) (width 0.2) (layer "F.Cu") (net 10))
 (segment (start 100 117.78) (end 101.78 117.78) (width 0.2) (layer "F.Cu") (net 10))
 (segment (start 104.5 121.9) (end 104.5 121) (width 0.2) (layer "F.Cu") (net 10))
 (via (at 101.8 117.8) (size 0.6) (drill 0.3) (layers "F.Cu" "B.Cu") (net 10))
 (via (at 104.5 121.9) (size 0.6) (drill 0.3) (layers "F.Cu" "B.Cu") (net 10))
 (segment (start 104.5 120.1) (end 104.5 121.9) (width 0.2) (layer "B.Cu") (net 10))
 (segment (start 101.8 117.8) (end 102.2 117.8) (width 0.2) (layer "B.Cu") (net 10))
 (segment (start 102.2 117.8) (end 104.5 120.1) (width 0.2) (layer "B.Cu") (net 10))
 (segment (start 100 112.7) (end 101.2 111.5) (width 0.2) (layer "F.Cu") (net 3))
 (segment (start 101.2 111.5) (end 104.5 111.5) (width 0.2) (layer "F.Cu") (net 3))
 (segment (start 101.74 113.5) (end 104.5 113.5) (width 0.2) (layer "F.Cu") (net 1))
 (segment (start 100 115.24) (end 101.74 113.5) (width 0.2) (layer "F.Cu") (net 1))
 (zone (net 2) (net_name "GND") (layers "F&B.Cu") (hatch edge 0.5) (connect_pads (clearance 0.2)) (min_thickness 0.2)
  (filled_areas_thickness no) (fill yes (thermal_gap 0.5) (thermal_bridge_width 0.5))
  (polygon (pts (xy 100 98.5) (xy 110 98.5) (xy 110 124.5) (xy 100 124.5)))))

